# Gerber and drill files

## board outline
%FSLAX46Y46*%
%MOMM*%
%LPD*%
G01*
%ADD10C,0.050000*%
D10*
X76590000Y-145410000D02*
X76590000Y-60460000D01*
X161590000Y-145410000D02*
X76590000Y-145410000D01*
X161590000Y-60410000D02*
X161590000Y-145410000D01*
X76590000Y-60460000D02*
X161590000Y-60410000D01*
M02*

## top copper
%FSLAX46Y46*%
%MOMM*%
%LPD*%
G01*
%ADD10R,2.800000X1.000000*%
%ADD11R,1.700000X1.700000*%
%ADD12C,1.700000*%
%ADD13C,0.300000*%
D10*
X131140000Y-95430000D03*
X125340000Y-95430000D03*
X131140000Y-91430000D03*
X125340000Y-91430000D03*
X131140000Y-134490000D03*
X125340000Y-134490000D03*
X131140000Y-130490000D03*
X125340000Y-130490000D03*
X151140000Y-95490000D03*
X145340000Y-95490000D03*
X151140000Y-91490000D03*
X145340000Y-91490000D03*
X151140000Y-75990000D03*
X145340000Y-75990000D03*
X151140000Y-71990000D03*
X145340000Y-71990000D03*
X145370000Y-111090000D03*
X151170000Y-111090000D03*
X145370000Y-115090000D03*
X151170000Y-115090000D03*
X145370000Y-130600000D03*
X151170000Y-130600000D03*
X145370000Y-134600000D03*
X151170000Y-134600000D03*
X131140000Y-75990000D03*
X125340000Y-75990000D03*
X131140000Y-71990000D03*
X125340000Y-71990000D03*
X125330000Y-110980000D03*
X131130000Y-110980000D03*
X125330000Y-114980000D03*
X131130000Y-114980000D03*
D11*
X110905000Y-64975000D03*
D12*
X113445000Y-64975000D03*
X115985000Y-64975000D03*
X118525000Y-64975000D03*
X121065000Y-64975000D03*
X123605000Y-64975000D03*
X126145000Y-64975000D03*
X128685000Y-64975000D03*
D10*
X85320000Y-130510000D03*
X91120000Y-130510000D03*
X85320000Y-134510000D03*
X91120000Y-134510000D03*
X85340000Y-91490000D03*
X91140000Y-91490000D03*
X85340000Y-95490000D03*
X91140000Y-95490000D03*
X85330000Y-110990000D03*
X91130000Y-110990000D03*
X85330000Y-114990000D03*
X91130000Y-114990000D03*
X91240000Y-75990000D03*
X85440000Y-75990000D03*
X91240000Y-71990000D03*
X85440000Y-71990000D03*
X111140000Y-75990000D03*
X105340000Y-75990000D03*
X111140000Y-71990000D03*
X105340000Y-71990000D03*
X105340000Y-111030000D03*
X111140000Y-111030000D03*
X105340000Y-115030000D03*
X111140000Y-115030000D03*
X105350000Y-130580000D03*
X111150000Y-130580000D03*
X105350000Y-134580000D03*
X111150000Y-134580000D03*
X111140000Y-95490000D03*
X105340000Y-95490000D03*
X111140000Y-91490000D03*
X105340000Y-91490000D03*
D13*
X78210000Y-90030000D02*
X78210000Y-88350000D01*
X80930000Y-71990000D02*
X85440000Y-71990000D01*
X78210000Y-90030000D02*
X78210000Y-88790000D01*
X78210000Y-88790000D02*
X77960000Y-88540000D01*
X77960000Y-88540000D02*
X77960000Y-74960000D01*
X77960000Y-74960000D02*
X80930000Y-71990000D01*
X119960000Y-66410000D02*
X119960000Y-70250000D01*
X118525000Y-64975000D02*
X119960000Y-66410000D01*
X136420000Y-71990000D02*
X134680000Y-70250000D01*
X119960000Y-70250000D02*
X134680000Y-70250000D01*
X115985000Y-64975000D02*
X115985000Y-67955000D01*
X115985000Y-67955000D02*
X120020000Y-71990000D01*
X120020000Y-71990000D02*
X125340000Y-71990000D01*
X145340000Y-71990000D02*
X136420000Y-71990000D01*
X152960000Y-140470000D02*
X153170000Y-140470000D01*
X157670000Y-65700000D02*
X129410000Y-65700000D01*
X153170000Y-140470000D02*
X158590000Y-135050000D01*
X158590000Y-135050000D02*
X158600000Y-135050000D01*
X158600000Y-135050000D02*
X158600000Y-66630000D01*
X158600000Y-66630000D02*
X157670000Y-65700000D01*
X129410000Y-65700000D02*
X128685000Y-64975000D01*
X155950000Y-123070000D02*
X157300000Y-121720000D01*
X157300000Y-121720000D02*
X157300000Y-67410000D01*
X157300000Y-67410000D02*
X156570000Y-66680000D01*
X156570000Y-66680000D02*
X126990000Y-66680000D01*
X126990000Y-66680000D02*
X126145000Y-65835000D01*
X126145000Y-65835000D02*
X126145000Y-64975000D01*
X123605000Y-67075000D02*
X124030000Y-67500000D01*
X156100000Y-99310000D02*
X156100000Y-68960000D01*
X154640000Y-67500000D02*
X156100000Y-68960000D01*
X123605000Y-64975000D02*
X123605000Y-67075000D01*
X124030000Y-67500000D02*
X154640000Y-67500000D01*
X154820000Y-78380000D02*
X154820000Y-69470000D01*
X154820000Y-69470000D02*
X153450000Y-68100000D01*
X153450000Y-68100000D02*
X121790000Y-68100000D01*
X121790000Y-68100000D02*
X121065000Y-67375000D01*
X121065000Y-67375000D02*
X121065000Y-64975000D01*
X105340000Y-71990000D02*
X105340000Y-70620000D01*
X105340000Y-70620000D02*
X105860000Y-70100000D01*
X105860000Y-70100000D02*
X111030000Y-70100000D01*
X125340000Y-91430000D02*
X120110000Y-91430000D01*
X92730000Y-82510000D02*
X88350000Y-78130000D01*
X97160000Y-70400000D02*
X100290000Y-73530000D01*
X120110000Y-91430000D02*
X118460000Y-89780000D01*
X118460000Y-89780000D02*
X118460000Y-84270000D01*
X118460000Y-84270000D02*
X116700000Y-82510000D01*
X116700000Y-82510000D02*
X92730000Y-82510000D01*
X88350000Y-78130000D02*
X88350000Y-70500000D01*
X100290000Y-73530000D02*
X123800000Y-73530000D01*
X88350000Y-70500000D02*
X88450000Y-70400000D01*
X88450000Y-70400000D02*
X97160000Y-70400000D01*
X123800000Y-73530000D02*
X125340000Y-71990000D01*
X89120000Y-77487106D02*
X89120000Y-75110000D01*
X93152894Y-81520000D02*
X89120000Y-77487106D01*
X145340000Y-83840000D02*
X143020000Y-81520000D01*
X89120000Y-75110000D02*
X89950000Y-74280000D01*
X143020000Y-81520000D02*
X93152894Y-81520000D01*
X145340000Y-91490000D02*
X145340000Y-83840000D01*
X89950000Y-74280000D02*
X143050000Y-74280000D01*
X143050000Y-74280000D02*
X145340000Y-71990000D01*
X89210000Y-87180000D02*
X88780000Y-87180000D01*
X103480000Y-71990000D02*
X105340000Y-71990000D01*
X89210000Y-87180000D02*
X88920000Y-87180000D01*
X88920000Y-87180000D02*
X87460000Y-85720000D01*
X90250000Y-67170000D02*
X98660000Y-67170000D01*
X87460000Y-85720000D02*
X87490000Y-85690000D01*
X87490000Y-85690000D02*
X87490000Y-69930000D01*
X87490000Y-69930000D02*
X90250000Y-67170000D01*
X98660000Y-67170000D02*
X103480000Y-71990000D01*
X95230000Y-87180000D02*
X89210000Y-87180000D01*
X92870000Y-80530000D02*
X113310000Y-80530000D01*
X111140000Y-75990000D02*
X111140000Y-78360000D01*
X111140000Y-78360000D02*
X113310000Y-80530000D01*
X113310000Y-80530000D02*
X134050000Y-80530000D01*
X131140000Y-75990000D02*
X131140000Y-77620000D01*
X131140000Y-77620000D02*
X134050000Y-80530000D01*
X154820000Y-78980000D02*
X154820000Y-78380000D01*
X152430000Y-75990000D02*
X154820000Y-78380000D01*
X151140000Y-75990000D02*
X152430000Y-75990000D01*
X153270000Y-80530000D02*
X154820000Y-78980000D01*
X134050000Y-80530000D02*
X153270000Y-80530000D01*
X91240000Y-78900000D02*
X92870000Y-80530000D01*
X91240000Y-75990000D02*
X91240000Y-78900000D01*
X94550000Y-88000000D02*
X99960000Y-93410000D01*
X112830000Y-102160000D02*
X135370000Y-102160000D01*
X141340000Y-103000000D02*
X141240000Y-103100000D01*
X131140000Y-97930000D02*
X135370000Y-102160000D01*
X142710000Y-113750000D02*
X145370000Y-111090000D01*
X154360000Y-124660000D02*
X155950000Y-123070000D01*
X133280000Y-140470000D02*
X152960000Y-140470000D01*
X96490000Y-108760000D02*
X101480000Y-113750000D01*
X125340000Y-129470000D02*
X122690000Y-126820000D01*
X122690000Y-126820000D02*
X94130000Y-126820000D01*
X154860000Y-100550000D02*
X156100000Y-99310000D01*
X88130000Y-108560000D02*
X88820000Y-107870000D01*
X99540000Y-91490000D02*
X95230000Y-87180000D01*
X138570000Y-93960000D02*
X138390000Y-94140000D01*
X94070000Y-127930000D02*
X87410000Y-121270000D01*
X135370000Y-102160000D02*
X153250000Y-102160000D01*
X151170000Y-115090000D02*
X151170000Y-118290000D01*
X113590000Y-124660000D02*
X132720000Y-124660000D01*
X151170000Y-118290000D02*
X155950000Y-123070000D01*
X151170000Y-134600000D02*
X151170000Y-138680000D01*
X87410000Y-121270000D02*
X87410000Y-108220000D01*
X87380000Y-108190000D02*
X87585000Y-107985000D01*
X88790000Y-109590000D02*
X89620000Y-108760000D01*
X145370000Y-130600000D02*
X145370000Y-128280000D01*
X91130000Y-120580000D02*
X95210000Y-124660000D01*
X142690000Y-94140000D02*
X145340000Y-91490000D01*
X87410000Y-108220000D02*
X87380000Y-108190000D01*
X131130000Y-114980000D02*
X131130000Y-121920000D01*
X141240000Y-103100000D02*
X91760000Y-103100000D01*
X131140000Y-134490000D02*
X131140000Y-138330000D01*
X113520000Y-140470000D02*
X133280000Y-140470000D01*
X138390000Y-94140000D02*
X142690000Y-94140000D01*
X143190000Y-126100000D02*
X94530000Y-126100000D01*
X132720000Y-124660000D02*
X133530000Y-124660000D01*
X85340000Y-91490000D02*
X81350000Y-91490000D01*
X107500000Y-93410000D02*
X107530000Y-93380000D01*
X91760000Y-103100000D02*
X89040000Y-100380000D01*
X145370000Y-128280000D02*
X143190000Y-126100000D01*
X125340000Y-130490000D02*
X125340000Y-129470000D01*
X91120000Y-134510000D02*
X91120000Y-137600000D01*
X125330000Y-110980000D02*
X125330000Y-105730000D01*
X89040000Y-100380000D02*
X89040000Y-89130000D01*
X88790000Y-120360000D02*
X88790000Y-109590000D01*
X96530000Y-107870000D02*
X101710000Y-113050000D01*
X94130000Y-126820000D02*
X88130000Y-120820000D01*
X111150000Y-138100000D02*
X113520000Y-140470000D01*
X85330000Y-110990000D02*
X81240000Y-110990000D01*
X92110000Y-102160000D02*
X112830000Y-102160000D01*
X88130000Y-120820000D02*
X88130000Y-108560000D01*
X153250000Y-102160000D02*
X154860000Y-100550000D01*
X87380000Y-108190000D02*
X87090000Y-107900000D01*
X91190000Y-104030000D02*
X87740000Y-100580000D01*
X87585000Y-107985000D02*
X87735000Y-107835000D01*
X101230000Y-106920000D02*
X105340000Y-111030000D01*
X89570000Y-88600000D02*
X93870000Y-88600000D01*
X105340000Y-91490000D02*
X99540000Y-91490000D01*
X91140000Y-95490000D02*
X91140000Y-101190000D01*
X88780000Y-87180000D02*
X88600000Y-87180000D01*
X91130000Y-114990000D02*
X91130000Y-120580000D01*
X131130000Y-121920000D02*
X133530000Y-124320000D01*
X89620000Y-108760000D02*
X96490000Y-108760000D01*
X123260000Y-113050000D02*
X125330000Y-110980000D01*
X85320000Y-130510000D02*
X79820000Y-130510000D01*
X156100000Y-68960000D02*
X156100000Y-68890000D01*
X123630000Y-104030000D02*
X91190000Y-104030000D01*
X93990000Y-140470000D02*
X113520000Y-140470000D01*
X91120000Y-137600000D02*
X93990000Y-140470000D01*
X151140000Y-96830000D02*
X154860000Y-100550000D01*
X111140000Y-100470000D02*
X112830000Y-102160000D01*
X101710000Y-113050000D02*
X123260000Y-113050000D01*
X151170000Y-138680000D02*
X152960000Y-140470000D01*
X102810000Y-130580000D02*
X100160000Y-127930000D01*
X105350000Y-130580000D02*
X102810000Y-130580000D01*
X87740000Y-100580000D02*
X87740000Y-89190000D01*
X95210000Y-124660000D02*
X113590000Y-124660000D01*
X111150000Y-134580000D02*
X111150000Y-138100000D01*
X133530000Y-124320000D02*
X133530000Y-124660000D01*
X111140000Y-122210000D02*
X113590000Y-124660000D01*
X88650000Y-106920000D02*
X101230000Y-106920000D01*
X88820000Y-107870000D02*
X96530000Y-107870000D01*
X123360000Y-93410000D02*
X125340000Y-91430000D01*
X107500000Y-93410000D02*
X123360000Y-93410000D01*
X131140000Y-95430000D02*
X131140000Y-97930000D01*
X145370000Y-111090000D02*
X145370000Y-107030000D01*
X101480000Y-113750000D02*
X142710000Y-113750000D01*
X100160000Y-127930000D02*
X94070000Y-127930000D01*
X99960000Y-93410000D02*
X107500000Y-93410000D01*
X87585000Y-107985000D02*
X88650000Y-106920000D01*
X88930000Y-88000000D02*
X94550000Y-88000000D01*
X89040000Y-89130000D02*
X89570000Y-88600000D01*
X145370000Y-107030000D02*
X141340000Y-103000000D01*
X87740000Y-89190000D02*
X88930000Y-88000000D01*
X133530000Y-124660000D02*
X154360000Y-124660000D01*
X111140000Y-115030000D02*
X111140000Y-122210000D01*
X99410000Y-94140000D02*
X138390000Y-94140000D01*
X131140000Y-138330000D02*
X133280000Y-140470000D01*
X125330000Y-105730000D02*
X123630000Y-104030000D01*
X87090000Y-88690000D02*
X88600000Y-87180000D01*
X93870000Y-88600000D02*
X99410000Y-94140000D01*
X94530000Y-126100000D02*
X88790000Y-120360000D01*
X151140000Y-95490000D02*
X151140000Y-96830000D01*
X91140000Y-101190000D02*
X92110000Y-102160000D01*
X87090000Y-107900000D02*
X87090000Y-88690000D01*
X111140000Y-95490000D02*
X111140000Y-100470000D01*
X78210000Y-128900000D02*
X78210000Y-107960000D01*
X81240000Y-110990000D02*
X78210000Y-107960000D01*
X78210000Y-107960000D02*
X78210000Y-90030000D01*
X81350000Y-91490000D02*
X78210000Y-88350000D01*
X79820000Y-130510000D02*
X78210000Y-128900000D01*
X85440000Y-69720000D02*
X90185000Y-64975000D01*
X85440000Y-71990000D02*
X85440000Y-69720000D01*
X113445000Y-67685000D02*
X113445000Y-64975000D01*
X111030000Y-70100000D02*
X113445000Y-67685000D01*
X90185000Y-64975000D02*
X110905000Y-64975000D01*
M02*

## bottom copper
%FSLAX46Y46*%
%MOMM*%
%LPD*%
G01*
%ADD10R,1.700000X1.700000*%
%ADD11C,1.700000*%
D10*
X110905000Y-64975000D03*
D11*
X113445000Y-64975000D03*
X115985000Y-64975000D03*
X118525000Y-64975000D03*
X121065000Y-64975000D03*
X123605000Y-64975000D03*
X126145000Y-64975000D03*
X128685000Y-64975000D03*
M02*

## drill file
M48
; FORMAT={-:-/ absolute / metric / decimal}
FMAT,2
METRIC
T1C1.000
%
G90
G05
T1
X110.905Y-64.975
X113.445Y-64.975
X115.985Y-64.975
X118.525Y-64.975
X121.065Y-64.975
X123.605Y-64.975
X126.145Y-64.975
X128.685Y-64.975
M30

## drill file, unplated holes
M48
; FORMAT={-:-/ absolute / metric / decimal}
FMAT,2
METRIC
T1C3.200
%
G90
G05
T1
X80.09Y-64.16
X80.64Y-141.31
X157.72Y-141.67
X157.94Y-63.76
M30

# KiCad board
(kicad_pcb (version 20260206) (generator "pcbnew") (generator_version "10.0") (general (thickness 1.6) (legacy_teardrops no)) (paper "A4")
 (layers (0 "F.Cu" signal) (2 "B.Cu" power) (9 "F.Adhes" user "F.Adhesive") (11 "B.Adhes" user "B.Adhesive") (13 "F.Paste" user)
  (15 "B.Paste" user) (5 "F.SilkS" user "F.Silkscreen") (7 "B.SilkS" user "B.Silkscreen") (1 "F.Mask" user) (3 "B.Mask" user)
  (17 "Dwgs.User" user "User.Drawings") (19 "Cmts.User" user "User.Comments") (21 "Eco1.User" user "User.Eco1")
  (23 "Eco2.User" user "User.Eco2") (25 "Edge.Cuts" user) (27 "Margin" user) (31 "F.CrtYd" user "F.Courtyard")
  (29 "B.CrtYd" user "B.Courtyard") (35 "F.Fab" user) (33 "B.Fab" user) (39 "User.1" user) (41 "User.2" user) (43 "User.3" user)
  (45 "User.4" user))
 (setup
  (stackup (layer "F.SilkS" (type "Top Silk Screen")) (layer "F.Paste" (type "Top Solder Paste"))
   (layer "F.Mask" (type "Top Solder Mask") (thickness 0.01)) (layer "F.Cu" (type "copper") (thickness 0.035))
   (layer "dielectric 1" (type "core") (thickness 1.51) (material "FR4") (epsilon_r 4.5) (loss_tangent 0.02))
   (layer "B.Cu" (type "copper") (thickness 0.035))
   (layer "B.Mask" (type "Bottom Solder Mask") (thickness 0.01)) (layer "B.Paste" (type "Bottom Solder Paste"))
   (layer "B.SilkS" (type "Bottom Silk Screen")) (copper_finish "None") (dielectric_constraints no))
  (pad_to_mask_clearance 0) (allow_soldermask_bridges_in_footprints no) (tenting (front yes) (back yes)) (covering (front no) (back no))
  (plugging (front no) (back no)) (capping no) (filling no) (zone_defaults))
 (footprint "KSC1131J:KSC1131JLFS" (layer "F.Cu") (at 128.24 93.43)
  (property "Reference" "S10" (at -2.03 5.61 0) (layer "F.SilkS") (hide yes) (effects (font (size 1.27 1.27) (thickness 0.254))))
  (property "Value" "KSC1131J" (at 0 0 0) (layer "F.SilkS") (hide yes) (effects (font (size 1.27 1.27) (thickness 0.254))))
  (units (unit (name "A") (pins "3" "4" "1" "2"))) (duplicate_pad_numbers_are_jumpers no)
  (pad "1" smd rect (at -2.9 -2 90) (size 1 2.8) (layers "F.Cu" "F.Mask" "F.Paste") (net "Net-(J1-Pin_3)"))
  (pad "2" smd rect (at 2.9 -2 90) (size 1 2.8) (layers "F.Cu" "F.Mask" "F.Paste") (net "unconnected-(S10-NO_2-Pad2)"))
  (pad "3" smd rect (at -2.9 2 90) (size 1 2.8) (layers "F.Cu" "F.Mask" "F.Paste") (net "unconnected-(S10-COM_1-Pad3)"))
  (pad "4" smd rect (at 2.9 2 90) (size 1 2.8) (layers "F.Cu" "F.Mask" "F.Paste") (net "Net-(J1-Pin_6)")))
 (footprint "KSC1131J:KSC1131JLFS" (layer "F.Cu") (at 148.24 73.99)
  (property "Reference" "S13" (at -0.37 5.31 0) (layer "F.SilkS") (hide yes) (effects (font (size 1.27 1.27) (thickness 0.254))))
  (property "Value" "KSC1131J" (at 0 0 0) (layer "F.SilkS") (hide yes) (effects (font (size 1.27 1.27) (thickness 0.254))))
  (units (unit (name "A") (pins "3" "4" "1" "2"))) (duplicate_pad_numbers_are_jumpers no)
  (pad "1" smd rect (at -2.9 -2 90) (size 1 2.8) (layers "F.Cu" "F.Mask" "F.Paste") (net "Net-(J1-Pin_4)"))
  (pad "2" smd rect (at 2.9 -2 90) (size 1 2.8) (layers "F.Cu" "F.Mask" "F.Paste") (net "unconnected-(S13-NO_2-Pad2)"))
  (pad "3" smd rect (at -2.9 2 90) (size 1 2.8) (layers "F.Cu" "F.Mask" "F.Paste") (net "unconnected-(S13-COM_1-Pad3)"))
  (pad "4" smd rect (at 2.9 2 90) (size 1 2.8) (layers "F.Cu" "F.Mask" "F.Paste") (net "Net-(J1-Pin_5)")))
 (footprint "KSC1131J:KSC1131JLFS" (layer "F.Cu") (at 108.24 73.99)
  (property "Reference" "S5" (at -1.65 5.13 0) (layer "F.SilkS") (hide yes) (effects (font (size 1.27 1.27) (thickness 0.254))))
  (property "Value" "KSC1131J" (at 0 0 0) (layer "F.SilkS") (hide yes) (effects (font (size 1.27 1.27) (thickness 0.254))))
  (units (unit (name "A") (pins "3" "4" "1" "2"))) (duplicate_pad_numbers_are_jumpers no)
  (pad "1" smd rect (at -2.9 -2 90) (size 1 2.8) (layers "F.Cu" "F.Mask" "F.Paste") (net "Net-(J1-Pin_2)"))
  (pad "2" smd rect (at 2.9 -2 90) (size 1 2.8) (layers "F.Cu" "F.Mask" "F.Paste") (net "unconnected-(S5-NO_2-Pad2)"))
  (pad "3" smd rect (at -2.9 2 90) (size 1 2.8) (layers "F.Cu" "F.Mask" "F.Paste") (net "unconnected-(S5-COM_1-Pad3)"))
  (pad "4" smd rect (at 2.9 2 90) (size 1 2.8) (layers "F.Cu" "F.Mask" "F.Paste") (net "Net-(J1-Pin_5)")))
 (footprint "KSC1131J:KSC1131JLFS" (layer "F.Cu") (at 88.34 73.99)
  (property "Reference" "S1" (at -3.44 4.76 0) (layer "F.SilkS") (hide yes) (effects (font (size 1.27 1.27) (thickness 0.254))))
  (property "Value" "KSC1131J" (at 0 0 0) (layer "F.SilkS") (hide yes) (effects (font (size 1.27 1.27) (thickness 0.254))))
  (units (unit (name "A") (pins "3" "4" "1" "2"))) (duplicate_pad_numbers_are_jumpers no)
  (pad "1" smd rect (at -2.9 -2 90) (size 1 2.8) (layers "F.Cu" "F.Mask" "F.Paste") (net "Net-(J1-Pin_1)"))
  (pad "2" smd rect (at 2.9 -2 90) (size 1 2.8) (layers "F.Cu" "F.Mask" "F.Paste") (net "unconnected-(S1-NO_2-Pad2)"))
  (pad "3" smd rect (at -2.9 2 90) (size 1 2.8) (layers "F.Cu" "F.Mask" "F.Paste") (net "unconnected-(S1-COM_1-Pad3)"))
  (pad "4" smd rect (at 2.9 2 90) (size 1 2.8) (layers "F.Cu" "F.Mask" "F.Paste") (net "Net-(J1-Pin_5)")))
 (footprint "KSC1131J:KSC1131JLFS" (layer "F.Cu") (at 148.27 132.6)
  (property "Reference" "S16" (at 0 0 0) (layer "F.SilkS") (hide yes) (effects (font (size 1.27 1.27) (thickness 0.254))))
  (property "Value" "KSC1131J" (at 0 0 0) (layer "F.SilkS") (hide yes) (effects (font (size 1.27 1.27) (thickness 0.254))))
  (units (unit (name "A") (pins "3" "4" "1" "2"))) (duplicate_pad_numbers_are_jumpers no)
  (pad "1" smd rect (at -2.9 -2 90) (size 1 2.8) (layers "F.Cu" "F.Mask" "F.Paste") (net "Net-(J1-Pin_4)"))
  (pad "2" smd rect (at 2.9 -2 90) (size 1 2.8) (layers "F.Cu" "F.Mask" "F.Paste") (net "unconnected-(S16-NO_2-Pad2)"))
  (pad "3" smd rect (at -2.9 2 90) (size 1 2.8) (layers "F.Cu" "F.Mask" "F.Paste") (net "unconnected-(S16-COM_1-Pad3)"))
  (pad "4" smd rect (at 2.9 2 90) (size 1 2.8) (layers "F.Cu" "F.Mask" "F.Paste") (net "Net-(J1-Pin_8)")))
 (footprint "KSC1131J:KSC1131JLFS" (layer "F.Cu") (at 128.24 73.99)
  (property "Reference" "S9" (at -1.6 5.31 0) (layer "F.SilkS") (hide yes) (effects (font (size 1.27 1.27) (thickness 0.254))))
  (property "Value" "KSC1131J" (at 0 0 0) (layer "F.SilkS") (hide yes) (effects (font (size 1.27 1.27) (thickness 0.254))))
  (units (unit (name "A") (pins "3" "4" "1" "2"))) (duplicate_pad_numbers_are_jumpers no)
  (pad "1" smd rect (at -2.9 -2 90) (size 1 2.8) (layers "F.Cu" "F.Mask" "F.Paste") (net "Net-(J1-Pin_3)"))
  (pad "2" smd rect (at 2.9 -2 90) (size 1 2.8) (layers "F.Cu" "F.Mask" "F.Paste") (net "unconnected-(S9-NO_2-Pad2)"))
  (pad "3" smd rect (at -2.9 2 90) (size 1 2.8) (layers "F.Cu" "F.Mask" "F.Paste") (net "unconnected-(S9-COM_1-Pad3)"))
  (pad "4" smd rect (at 2.9 2 90) (size 1 2.8) (layers "F.Cu" "F.Mask" "F.Paste") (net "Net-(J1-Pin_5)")))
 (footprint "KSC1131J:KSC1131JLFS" (layer "F.Cu") (at 108.24 93.49)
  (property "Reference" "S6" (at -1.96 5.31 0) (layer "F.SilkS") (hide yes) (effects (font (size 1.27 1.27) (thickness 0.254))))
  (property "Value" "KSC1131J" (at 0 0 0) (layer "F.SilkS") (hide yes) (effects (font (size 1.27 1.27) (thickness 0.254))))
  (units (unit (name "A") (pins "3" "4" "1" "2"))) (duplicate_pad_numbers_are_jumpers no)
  (pad "1" smd rect (at -2.9 -2 90) (size 1 2.8) (layers "F.Cu" "F.Mask" "F.Paste") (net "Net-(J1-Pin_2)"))
  (pad "2" smd rect (at 2.9 -2 90) (size 1 2.8) (layers "F.Cu" "F.Mask" "F.Paste") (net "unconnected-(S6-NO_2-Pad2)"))
  (pad "3" smd rect (at -2.9 2 90) (size 1 2.8) (layers "F.Cu" "F.Mask" "F.Paste") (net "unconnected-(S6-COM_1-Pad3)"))
  (pad "4" smd rect (at 2.9 2 90) (size 1 2.8) (layers "F.Cu" "F.Mask" "F.Paste") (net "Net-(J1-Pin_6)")))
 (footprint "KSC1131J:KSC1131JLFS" (layer "F.Cu") (at 148.27 113.09)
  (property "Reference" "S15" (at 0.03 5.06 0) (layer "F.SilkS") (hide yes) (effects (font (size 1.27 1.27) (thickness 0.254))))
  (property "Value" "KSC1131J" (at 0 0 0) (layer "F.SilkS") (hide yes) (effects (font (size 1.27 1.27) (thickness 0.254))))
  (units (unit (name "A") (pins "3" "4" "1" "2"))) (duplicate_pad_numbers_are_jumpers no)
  (pad "1" smd rect (at -2.9 -2 90) (size 1 2.8) (layers "F.Cu" "F.Mask" "F.Paste") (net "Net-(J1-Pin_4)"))
  (pad "2" smd rect (at 2.9 -2 90) (size 1 2.8) (layers "F.Cu" "F.Mask" "F.Paste") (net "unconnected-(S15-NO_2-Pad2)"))
  (pad "3" smd rect (at -2.9 2 90) (size 1 2.8) (layers "F.Cu" "F.Mask" "F.Paste") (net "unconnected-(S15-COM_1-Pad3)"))
  (pad "4" smd rect (at 2.9 2 90) (size 1 2.8) (layers "F.Cu" "F.Mask" "F.Paste") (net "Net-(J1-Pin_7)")))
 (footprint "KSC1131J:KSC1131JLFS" (layer "F.Cu") (at 108.24 113.03)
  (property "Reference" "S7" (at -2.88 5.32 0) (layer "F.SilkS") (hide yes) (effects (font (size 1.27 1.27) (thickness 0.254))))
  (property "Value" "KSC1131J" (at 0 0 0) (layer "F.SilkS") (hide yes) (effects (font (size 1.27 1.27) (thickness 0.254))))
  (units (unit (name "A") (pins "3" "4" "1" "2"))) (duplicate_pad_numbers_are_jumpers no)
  (pad "1" smd rect (at -2.9 -2 90) (size 1 2.8) (layers "F.Cu" "F.Mask" "F.Paste") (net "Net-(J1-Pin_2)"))
  (pad "2" smd rect (at 2.9 -2 90) (size 1 2.8) (layers "F.Cu" "F.Mask" "F.Paste") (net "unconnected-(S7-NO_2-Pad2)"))
  (pad "3" smd rect (at -2.9 2 90) (size 1 2.8) (layers "F.Cu" "F.Mask" "F.Paste") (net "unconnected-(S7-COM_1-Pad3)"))
  (pad "4" smd rect (at 2.9 2 90) (size 1 2.8) (layers "F.Cu" "F.Mask" "F.Paste") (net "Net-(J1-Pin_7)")))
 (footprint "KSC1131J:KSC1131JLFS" (layer "F.Cu") (at 148.24 93.49)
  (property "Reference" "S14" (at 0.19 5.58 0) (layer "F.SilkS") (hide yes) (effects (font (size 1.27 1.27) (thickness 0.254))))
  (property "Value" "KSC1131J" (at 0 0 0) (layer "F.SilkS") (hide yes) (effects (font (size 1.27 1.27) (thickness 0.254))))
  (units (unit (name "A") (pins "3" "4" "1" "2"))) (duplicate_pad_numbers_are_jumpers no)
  (pad "1" smd rect (at -2.9 -2 90) (size 1 2.8) (layers "F.Cu" "F.Mask" "F.Paste") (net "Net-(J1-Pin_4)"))
  (pad "2" smd rect (at 2.9 -2 90) (size 1 2.8) (layers "F.Cu" "F.Mask" "F.Paste") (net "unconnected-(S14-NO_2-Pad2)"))
  (pad "3" smd rect (at -2.9 2 90) (size 1 2.8) (layers "F.Cu" "F.Mask" "F.Paste") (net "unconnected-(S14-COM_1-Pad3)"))
  (pad "4" smd rect (at 2.9 2 90) (size 1 2.8) (layers "F.Cu" "F.Mask" "F.Paste") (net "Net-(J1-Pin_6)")))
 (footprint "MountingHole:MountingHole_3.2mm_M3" (layer "F.Cu") (at 157.72 141.67)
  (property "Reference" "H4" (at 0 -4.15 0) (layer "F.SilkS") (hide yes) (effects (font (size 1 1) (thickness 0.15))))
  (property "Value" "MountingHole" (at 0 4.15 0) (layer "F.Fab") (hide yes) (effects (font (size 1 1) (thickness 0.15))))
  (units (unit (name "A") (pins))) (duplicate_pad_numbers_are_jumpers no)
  (pad "" np_thru_hole circle (at 0 0) (size 3.2 3.2) (drill 3.2) (layers "*.Cu" "*.Mask")))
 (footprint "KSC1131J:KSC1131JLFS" (layer "F.Cu") (at 128.24 132.49)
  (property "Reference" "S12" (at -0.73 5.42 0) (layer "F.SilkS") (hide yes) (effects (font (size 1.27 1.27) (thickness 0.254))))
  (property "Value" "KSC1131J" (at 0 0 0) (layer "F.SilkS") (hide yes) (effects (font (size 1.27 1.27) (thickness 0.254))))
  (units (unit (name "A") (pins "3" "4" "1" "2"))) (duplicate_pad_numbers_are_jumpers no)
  (pad "1" smd rect (at -2.9 -2 90) (size 1 2.8) (layers "F.Cu" "F.Mask" "F.Paste") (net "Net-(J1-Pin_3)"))
  (pad "2" smd rect (at 2.9 -2 90) (size 1 2.8) (layers "F.Cu" "F.Mask" "F.Paste") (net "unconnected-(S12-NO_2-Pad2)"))
  (pad "3" smd rect (at -2.9 2 90) (size 1 2.8) (layers "F.Cu" "F.Mask" "F.Paste") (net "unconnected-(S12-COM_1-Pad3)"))
  (pad "4" smd rect (at 2.9 2 90) (size 1 2.8) (layers "F.Cu" "F.Mask" "F.Paste") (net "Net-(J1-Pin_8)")))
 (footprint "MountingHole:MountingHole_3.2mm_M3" (layer "F.Cu") (at 157.94 63.76)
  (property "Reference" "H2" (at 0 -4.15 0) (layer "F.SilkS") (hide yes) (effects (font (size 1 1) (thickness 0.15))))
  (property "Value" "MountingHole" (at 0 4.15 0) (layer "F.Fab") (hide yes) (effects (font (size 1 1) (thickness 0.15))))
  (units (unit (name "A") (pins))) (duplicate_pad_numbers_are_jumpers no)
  (pad "" np_thru_hole circle (at 0 0) (size 3.2 3.2) (drill 3.2) (layers "*.Cu" "*.Mask")))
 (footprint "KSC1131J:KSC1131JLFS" (layer "F.Cu") (at 88.23 112.99)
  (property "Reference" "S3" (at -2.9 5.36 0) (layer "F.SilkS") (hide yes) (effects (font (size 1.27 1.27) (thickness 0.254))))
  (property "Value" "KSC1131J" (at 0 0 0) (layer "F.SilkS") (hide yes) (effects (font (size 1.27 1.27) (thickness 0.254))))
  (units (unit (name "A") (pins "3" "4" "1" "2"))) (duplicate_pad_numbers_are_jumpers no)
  (pad "1" smd rect (at -2.9 -2 90) (size 1 2.8) (layers "F.Cu" "F.Mask" "F.Paste") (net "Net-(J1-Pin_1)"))
  (pad "2" smd rect (at 2.9 -2 90) (size 1 2.8) (layers "F.Cu" "F.Mask" "F.Paste") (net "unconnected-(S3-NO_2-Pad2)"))
  (pad "3" smd rect (at -2.9 2 90) (size 1 2.8) (layers "F.Cu" "F.Mask" "F.Paste") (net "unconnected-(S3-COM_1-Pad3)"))
  (pad "4" smd rect (at 2.9 2 90) (size 1 2.8) (layers "F.Cu" "F.Mask" "F.Paste") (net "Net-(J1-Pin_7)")))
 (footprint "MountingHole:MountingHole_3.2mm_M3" (layer "F.Cu") (at 80.64 141.31)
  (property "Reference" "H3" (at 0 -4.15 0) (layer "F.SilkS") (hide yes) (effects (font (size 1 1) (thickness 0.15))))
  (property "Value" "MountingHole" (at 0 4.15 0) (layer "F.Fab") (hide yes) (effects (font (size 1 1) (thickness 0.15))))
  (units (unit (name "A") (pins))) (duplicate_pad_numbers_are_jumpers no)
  (pad "" np_thru_hole circle (at 0 0) (size 3.2 3.2) (drill 3.2) (layers "*.Cu" "*.Mask")))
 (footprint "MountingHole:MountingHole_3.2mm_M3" (layer "F.Cu") (at 80.09 64.16)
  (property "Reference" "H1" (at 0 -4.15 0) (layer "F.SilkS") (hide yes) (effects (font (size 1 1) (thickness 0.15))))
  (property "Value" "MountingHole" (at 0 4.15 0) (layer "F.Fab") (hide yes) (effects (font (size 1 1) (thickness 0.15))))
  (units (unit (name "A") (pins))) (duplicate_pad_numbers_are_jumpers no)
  (pad "" np_thru_hole circle (at 0 0) (size 3.2 3.2) (drill 3.2) (layers "*.Cu" "*.Mask")))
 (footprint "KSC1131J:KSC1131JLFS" (layer "F.Cu") (at 88.24 93.49)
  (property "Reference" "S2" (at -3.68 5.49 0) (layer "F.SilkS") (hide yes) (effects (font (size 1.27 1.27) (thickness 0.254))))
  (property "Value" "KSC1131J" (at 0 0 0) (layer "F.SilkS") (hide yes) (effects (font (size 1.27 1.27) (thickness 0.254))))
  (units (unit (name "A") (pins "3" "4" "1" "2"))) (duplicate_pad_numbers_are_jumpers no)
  (pad "1" smd rect (at -2.9 -2 90) (size 1 2.8) (layers "F.Cu" "F.Mask" "F.Paste") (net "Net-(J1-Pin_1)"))
  (pad "2" smd rect (at 2.9 -2 90) (size 1 2.8) (layers "F.Cu" "F.Mask" "F.Paste") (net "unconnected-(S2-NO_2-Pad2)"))
  (pad "3" smd rect (at -2.9 2 90) (size 1 2.8) (layers "F.Cu" "F.Mask" "F.Paste") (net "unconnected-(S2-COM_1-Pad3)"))
  (pad "4" smd rect (at 2.9 2 90) (size 1 2.8) (layers "F.Cu" "F.Mask" "F.Paste") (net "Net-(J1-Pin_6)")))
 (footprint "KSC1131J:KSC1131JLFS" (layer "F.Cu") (at 128.23 112.98)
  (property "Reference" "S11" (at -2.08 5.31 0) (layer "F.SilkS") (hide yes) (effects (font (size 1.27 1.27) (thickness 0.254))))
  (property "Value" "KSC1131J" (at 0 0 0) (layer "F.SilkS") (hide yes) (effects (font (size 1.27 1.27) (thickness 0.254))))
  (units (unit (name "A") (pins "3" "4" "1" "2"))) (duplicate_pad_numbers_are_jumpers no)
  (pad "1" smd rect (at -2.9 -2 90) (size 1 2.8) (layers "F.Cu" "F.Mask" "F.Paste") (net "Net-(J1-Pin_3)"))
  (pad "2" smd rect (at 2.9 -2 90) (size 1 2.8) (layers "F.Cu" "F.Mask" "F.Paste") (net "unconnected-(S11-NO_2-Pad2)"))
  (pad "3" smd rect (at -2.9 2 90) (size 1 2.8) (layers "F.Cu" "F.Mask" "F.Paste") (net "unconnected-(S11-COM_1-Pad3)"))
  (pad "4" smd rect (at 2.9 2 90) (size 1 2.8) (layers "F.Cu" "F.Mask" "F.Paste") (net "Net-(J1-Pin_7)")))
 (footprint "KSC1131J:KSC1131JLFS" (layer "F.Cu") (at 88.22 132.51)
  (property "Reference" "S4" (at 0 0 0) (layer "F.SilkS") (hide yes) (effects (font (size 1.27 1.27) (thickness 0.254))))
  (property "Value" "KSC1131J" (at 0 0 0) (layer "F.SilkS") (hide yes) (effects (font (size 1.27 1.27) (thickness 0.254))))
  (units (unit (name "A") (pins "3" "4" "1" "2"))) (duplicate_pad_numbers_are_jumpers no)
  (pad "1" smd rect (at -2.9 -2 90) (size 1 2.8) (layers "F.Cu" "F.Mask" "F.Paste") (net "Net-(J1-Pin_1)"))
  (pad "2" smd rect (at 2.9 -2 90) (size 1 2.8) (layers "F.Cu" "F.Mask" "F.Paste") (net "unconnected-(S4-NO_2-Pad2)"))
  (pad "3" smd rect (at -2.9 2 90) (size 1 2.8) (layers "F.Cu" "F.Mask" "F.Paste") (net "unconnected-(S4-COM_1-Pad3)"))
  (pad "4" smd rect (at 2.9 2 90) (size 1 2.8) (layers "F.Cu" "F.Mask" "F.Paste") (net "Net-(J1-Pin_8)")))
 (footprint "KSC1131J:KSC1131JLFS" (layer "F.Cu") (at 108.25 132.58)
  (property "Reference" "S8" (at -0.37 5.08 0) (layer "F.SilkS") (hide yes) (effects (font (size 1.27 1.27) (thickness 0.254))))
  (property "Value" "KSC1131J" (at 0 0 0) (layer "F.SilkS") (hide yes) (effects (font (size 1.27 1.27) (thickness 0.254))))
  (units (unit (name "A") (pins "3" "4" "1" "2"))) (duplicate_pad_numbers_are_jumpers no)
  (pad "1" smd rect (at -2.9 -2 90) (size 1 2.8) (layers "F.Cu" "F.Mask" "F.Paste") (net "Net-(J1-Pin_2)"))
  (pad "2" smd rect (at 2.9 -2 90) (size 1 2.8) (layers "F.Cu" "F.Mask" "F.Paste") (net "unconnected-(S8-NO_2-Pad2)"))
  (pad "3" smd rect (at -2.9 2 90) (size 1 2.8) (layers "F.Cu" "F.Mask" "F.Paste") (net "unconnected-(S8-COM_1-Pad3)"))
  (pad "4" smd rect (at 2.9 2 90) (size 1 2.8) (layers "F.Cu" "F.Mask" "F.Paste") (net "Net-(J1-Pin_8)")))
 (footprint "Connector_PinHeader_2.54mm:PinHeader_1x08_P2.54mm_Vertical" (layer "F.Cu") (at 110.905 64.975 90)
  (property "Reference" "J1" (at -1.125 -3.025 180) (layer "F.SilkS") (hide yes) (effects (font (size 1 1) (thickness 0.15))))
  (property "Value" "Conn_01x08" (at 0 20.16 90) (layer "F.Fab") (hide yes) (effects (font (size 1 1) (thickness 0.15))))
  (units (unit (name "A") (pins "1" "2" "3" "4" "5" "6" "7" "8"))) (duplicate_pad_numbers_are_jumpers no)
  (pad "1" thru_hole rect (at 0 0 90) (size 1.7 1.7) (drill 1) (layers "*.Cu" "*.Mask") (remove_unused_layers no) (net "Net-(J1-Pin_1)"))
  (pad "2" thru_hole circle (at 0 2.54 90) (size 1.7 1.7) (drill 1) (layers "*.Cu" "*.Mask") (remove_unused_layers no)
   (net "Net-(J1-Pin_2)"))
  (pad "3" thru_hole circle (at 0 5.08 90) (size 1.7 1.7) (drill 1) (layers "*.Cu" "*.Mask") (remove_unused_layers no)
   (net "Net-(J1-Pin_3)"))
  (pad "4" thru_hole circle (at 0 7.62 90) (size 1.7 1.7) (drill 1) (layers "*.Cu" "*.Mask") (remove_unused_layers no)
   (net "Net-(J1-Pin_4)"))
  (pad "5" thru_hole circle (at 0 10.16 90) (size 1.7 1.7) (drill 1) (layers "*.Cu" "*.Mask") (remove_unused_layers no)
   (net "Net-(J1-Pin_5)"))
  (pad "6" thru_hole circle (at 0 12.7 90) (size 1.7 1.7) (drill 1) (layers "*.Cu" "*.Mask") (remove_unused_layers no)
   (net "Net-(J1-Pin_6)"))
  (pad "7" thru_hole circle (at 0 15.24 90) (size 1.7 1.7) (drill 1) (layers "*.Cu" "*.Mask") (remove_unused_layers no)
   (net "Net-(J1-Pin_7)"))
  (pad "8" thru_hole circle (at 0 17.78 90) (size 1.7 1.7) (drill 1) (layers "*.Cu" "*.Mask") (remove_unused_layers no)
   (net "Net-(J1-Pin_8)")))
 (gr_line (start 76.59 60.46) (end 161.59 60.41) (stroke (width 0.05) (type default)) (layer "Edge.Cuts"))
 (gr_line (start 76.59 145.41) (end 76.59 60.46) (stroke (width 0.05) (type default)) (layer "Edge.Cuts"))
 (gr_line (start 161.59 60.41) (end 161.59 145.41) (stroke (width 0.05) (type default)) (layer "Edge.Cuts"))
 (gr_line (start 161.59 145.41) (end 76.59 145.41) (stroke (width 0.05) (type default)) (layer "Edge.Cuts"))
 (segment (start 85.34 91.49) (end 81.35 91.49) (width 0.3) (layer "F.Cu") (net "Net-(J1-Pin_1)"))
 (segment (start 85.44 69.72) (end 90.185 64.975) (width 0.3) (layer "F.Cu") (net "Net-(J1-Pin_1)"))
 (segment (start 79.82 130.51) (end 78.21 128.9) (width 0.3) (layer "F.Cu") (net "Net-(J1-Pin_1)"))
 (segment (start 78.21 128.9) (end 78.21 107.96) (width 0.3) (layer "F.Cu") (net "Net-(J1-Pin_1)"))
 (segment (start 85.33 110.99) (end 81.24 110.99) (width 0.3) (layer "F.Cu") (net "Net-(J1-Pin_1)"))
 (segment (start 78.21 88.79) (end 77.96 88.54) (width 0.3) (layer "F.Cu") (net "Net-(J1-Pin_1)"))
 (segment (start 85.32 130.51) (end 79.82 130.51) (width 0.3) (layer "F.Cu") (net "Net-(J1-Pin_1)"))
 (segment (start 77.96 88.54) (end 77.96 74.96) (width 0.3) (layer "F.Cu") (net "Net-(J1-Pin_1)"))
 (segment (start 81.35 91.49) (end 78.21 88.35) (width 0.3) (layer "F.Cu") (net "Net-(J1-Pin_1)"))
 (segment (start 78.21 90.03) (end 78.21 88.79) (width 0.3) (layer "F.Cu") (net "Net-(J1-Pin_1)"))
 (segment (start 78.21 107.96) (end 78.21 90.03) (width 0.3) (layer "F.Cu") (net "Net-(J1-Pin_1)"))
 (segment (start 80.93 71.99) (end 85.44 71.99) (width 0.3) (layer "F.Cu") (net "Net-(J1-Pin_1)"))
 (segment (start 90.185 64.975) (end 110.905 64.975) (width 0.3) (layer "F.Cu") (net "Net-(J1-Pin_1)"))
 (segment (start 78.21 90.03) (end 78.21 88.35) (width 0.3) (layer "F.Cu") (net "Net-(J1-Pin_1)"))
 (segment (start 77.96 74.96) (end 80.93 71.99) (width 0.3) (layer "F.Cu") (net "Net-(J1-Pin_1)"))
 (segment (start 81.24 110.99) (end 78.21 107.96) (width 0.3) (layer "F.Cu") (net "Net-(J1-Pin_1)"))
 (segment (start 85.44 71.99) (end 85.44 69.72) (width 0.3) (layer "F.Cu") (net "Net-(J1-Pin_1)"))
 (segment (start 87.09 107.9) (end 87.09 88.69) (width 0.3) (layer "F.Cu") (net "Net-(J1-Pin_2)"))
 (segment (start 87.41 121.27) (end 87.41 108.22) (width 0.3) (layer "F.Cu") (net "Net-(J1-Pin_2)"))
 (segment (start 87.585 107.985) (end 87.735 107.835) (width 0.3) (layer "F.Cu") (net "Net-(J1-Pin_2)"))
 (segment (start 113.445 67.685) (end 113.445 64.975) (width 0.3) (layer "F.Cu") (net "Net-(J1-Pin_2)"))
 (segment (start 90.25 67.17) (end 98.66 67.17) (width 0.3) (layer "F.Cu") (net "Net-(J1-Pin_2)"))
 (segment (start 89.21 87.18) (end 88.78 87.18) (width 0.3) (layer "F.Cu") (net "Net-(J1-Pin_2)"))
 (segment (start 88.78 87.18) (end 88.6 87.18) (width 0.3) (layer "F.Cu") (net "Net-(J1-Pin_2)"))
 (segment (start 103.48 71.99) (end 105.34 71.99) (width 0.3) (layer "F.Cu") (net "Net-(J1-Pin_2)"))
 (segment (start 87.585 107.985) (end 88.65 106.92) (width 0.3) (layer "F.Cu") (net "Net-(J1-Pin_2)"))
 (segment (start 94.07 127.93) (end 87.41 121.27) (width 0.3) (layer "F.Cu") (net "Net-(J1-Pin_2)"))
 (segment (start 102.81 130.58) (end 100.16 127.93) (width 0.3) (layer "F.Cu") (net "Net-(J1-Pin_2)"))
 (segment (start 111.03 70.1) (end 113.445 67.685) (width 0.3) (layer "F.Cu") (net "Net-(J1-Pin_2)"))
 (segment (start 87.38 108.19) (end 87.09 107.9) (width 0.3) (layer "F.Cu") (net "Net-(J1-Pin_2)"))
 (segment (start 105.35 130.58) (end 102.81 130.58) (width 0.3) (layer "F.Cu") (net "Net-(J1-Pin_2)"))
 (segment (start 89.21 87.18) (end 88.92 87.18) (width 0.3) (layer "F.Cu") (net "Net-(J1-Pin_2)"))
 (segment (start 101.23 106.92) (end 105.34 111.03) (width 0.3) (layer "F.Cu") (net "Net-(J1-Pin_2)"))
 (segment (start 88.65 106.92) (end 101.23 106.92) (width 0.3) (layer "F.Cu") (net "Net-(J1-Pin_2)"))
 (segment (start 87.49 85.69) (end 87.49 69.93) (width 0.3) (layer "F.Cu") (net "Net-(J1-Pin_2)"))
 (segment (start 105.86 70.1) (end 111.03 70.1) (width 0.3) (layer "F.Cu") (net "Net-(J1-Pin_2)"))
 (segment (start 100.16 127.93) (end 94.07 127.93) (width 0.3) (layer "F.Cu") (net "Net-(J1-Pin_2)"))
 (segment (start 87.41 108.22) (end 87.38 108.19) (width 0.3) (layer "F.Cu") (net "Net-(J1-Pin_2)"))
 (segment (start 87.49 69.93) (end 90.25 67.17) (width 0.3) (layer "F.Cu") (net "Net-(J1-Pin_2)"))
 (segment (start 87.09 88.69) (end 88.6 87.18) (width 0.3) (layer "F.Cu") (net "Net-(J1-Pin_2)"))
 (segment (start 99.54 91.49) (end 95.23 87.18) (width 0.3) (layer "F.Cu") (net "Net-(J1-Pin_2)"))
 (segment (start 105.34 91.49) (end 99.54 91.49) (width 0.3) (layer "F.Cu") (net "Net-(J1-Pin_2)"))
 (segment (start 105.34 70.62) (end 105.86 70.1) (width 0.3) (layer "F.Cu") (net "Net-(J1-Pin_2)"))
 (segment (start 98.66 67.17) (end 103.48 71.99) (width 0.3) (layer "F.Cu") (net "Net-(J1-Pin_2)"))
 (segment (start 87.46 85.72) (end 87.49 85.69) (width 0.3) (layer "F.Cu") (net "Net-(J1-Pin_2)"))
 (segment (start 105.34 71.99) (end 105.34 70.62) (width 0.3) (layer "F.Cu") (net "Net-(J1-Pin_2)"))
 (segment (start 87.38 108.19) (end 87.585 107.985) (width 0.3) (layer "F.Cu") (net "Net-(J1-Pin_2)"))
 (segment (start 88.92 87.18) (end 87.46 85.72) (width 0.3) (layer "F.Cu") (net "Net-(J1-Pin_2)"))
 (segment (start 95.23 87.18) (end 89.21 87.18) (width 0.3) (layer "F.Cu") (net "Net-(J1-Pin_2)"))
 (segment (start 92.73 82.51) (end 88.35 78.13) (width 0.3) (layer "F.Cu") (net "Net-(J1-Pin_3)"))
 (segment (start 88.82 107.87) (end 96.53 107.87) (width 0.3) (layer "F.Cu") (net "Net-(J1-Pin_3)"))
 (segment (start 88.93 88) (end 94.55 88) (width 0.3) (layer "F.Cu") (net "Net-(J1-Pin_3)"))
 (segment (start 125.34 130.49) (end 125.34 129.47) (width 0.3) (layer "F.Cu") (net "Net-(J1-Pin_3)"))
 (segment (start 118.46 84.27) (end 116.7 82.51) (width 0.3) (layer "F.Cu") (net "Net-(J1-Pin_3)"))
 (segment (start 120.02 71.99) (end 125.34 71.99) (width 0.3) (layer "F.Cu") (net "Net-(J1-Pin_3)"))
 (segment (start 94.55 88) (end 99.96 93.41) (width 0.3) (layer "F.Cu") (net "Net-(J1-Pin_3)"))
 (segment (start 96.53 107.87) (end 101.71 113.05) (width 0.3) (layer "F.Cu") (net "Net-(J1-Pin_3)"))
 (segment (start 88.35 70.5) (end 88.45 70.4) (width 0.3) (layer "F.Cu") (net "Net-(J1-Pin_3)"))
 (segment (start 115.985 64.975) (end 115.985 67.955) (width 0.3) (layer "F.Cu") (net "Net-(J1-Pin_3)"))
 (segment (start 115.985 67.955) (end 120.02 71.99) (width 0.3) (layer "F.Cu") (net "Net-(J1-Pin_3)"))
 (segment (start 122.69 126.82) (end 94.13 126.82) (width 0.3) (layer "F.Cu") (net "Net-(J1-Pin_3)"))
 (segment (start 125.34 91.43) (end 120.11 91.43) (width 0.3) (layer "F.Cu") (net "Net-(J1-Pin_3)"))
 (segment (start 107.5 93.41) (end 107.53 93.38) (width 0.3) (layer "F.Cu") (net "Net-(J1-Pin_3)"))
 (segment (start 88.45 70.4) (end 97.16 70.4) (width 0.3) (layer "F.Cu") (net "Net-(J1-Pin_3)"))
 (segment (start 118.46 89.78) (end 118.46 84.27) (width 0.3) (layer "F.Cu") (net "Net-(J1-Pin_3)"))
 (segment (start 99.96 93.41) (end 107.5 93.41) (width 0.3) (layer "F.Cu") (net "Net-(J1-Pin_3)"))
 (segment (start 88.35 78.13) (end 88.35 70.5) (width 0.3) (layer "F.Cu") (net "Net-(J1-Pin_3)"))
 (segment (start 123.26 113.05) (end 125.33 110.98) (width 0.3) (layer "F.Cu") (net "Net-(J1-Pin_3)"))
 (segment (start 94.13 126.82) (end 88.13 120.82) (width 0.3) (layer "F.Cu") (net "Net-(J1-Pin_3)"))
 (segment (start 123.36 93.41) (end 125.34 91.43) (width 0.3) (layer "F.Cu") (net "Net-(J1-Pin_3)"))
 (segment (start 91.19 104.03) (end 87.74 100.58) (width 0.3) (layer "F.Cu") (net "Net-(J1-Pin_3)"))
 (segment (start 125.34 129.47) (end 122.69 126.82) (width 0.3) (layer "F.Cu") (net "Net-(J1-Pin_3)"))
 (segment (start 88.13 120.82) (end 88.13 108.56) (width 0.3) (layer "F.Cu") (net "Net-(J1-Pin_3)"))
 (segment (start 107.5 93.41) (end 123.36 93.41) (width 0.3) (layer "F.Cu") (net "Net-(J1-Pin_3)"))
 (segment (start 101.71 113.05) (end 123.26 113.05) (width 0.3) (layer "F.Cu") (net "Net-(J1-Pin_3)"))
 (segment (start 87.74 100.58) (end 87.74 89.19) (width 0.3) (layer "F.Cu") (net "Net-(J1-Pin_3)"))
 (segment (start 123.8 73.53) (end 125.34 71.99) (width 0.3) (layer "F.Cu") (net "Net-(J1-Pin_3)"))
 (segment (start 116.7 82.51) (end 92.73 82.51) (width 0.3) (layer "F.Cu") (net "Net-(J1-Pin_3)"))
 (segment (start 125.33 105.73) (end 123.63 104.03) (width 0.3) (layer "F.Cu") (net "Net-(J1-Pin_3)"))
 (segment (start 87.74 89.19) (end 88.93 88) (width 0.3) (layer "F.Cu") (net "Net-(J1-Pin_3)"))
 (segment (start 97.16 70.4) (end 100.29 73.53) (width 0.3) (layer "F.Cu") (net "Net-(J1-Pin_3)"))
 (segment (start 88.13 108.56) (end 88.82 107.87) (width 0.3) (layer "F.Cu") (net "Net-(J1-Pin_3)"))
 (segment (start 125.33 110.98) (end 125.33 105.73) (width 0.3) (layer "F.Cu") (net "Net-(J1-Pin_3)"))
 (segment (start 120.11 91.43) (end 118.46 89.78) (width 0.3) (layer "F.Cu") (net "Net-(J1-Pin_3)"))
 (segment (start 123.63 104.03) (end 91.19 104.03) (width 0.3) (layer "F.Cu") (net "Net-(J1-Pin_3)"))
 (segment (start 100.29 73.53) (end 123.8 73.53) (width 0.3) (layer "F.Cu") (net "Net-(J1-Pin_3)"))
 (segment (start 91.24 75.99) (end 91.24 78.9) (width 0.3) (layer "F.Cu") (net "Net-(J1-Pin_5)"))
 (segment (start 121.79 68.1) (end 121.065 67.375) (width 0.3) (layer "F.Cu") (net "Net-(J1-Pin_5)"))
 (segment (start 131.14 77.62) (end 134.05 80.53) (width 0.3) (layer "F.Cu") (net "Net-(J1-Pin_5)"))
 (segment (start 121.065 67.375) (end 121.065 64.975) (width 0.3) (layer "F.Cu") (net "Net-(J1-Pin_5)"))
 (segment (start 154.82 78.98) (end 154.82 78.38) (width 0.3) (layer "F.Cu") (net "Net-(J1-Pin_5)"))
 (segment (start 154.82 69.47) (end 153.45 68.1) (width 0.3) (layer "F.Cu") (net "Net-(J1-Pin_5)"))
 (segment (start 111.14 78.36) (end 113.31 80.53) (width 0.3) (layer "F.Cu") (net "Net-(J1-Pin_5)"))
 (segment (start 113.31 80.53) (end 134.05 80.53) (width 0.3) (layer "F.Cu") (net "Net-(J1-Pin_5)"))
 (segment (start 91.24 78.9) (end 92.87 80.53) (width 0.3) (layer "F.Cu") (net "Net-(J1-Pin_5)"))
 (segment (start 92.87 80.53) (end 113.31 80.53) (width 0.3) (layer "F.Cu") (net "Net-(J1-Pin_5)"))
 (segment (start 134.05 80.53) (end 153.27 80.53) (width 0.3) (layer "F.Cu") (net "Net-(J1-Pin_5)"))
 (segment (start 153.27 80.53) (end 154.82 78.98) (width 0.3) (layer "F.Cu") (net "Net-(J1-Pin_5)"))
 (segment (start 154.82 78.38) (end 154.82 69.47) (width 0.3) (layer "F.Cu") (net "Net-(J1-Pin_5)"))
 (segment (start 131.14 75.99) (end 131.14 77.62) (width 0.3) (layer "F.Cu") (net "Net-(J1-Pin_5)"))
 (segment (start 153.45 68.1) (end 121.79 68.1) (width 0.3) (layer "F.Cu") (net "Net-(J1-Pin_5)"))
 (segment (start 111.14 75.99) (end 111.14 78.36) (width 0.3) (layer "F.Cu") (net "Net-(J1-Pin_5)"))
 (segment (start 151.14 75.99) (end 152.43 75.99) (width 0.3) (layer "F.Cu") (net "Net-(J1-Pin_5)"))
 (segment (start 152.43 75.99) (end 154.82 78.38) (width 0.3) (layer "F.Cu") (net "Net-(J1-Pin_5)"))
 (segment (start 112.83 102.16) (end 135.37 102.16) (width 0.3) (layer "F.Cu") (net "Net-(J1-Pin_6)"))
 (segment (start 124.03 67.5) (end 154.64 67.5) (width 0.3) (layer "F.Cu") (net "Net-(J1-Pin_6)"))
 (segment (start 153.25 102.16) (end 154.86 100.55) (width 0.3) (layer "F.Cu") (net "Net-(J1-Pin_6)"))
 (segment (start 91.14 95.49) (end 91.14 101.19) (width 0.3) (layer "F.Cu") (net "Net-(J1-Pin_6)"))
 (segment (start 111.14 100.47) (end 112.83 102.16) (width 0.3) (layer "F.Cu") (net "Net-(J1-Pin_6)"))
 (segment (start 123.605 67.075) (end 124.03 67.5) (width 0.3) (layer "F.Cu") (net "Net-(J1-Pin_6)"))
 (segment (start 151.14 96.83) (end 154.86 100.55) (width 0.3) (layer "F.Cu") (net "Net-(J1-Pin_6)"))
 (segment (start 135.37 102.16) (end 153.25 102.16) (width 0.3) (layer "F.Cu") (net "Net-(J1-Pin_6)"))
 (segment (start 123.605 64.975) (end 123.605 67.075) (width 0.3) (layer "F.Cu") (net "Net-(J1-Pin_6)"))
 (segment (start 92.11 102.16) (end 112.83 102.16) (width 0.3) (layer "F.Cu") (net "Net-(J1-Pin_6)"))
 (segment (start 154.86 100.55) (end 156.1 99.31) (width 0.3) (layer "F.Cu") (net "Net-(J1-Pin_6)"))
 (segment (start 151.14 95.49) (end 151.14 96.83) (width 0.3) (layer "F.Cu") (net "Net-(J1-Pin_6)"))
 (segment (start 154.64 67.5) (end 156.1 68.96) (width 0.3) (layer "F.Cu") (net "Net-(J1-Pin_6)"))
 (segment (start 111.14 95.49) (end 111.14 100.47) (width 0.3) (layer "F.Cu") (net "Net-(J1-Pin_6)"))
 (segment (start 131.14 97.93) (end 135.37 102.16) (width 0.3) (layer "F.Cu") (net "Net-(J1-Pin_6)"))
 (segment (start 91.14 101.19) (end 92.11 102.16) (width 0.3) (layer "F.Cu") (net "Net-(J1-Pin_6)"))
 (segment (start 131.14 95.43) (end 131.14 97.93) (width 0.3) (layer "F.Cu") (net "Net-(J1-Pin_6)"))
 (segment (start 156.1 99.31) (end 156.1 68.96) (width 0.3) (layer "F.Cu") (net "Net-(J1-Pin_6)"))
 (segment (start 156.1 68.96) (end 156.1 68.89) (width 0.3) (layer "F.Cu") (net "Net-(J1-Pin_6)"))
 (segment (start 95.21 124.66) (end 113.59 124.66) (width 0.3) (layer "F.Cu") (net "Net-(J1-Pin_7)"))
 (segment (start 132.72 124.66) (end 133.53 124.66) (width 0.3) (layer "F.Cu") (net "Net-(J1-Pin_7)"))
 (segment (start 91.13 120.58) (end 95.21 124.66) (width 0.3) (layer "F.Cu") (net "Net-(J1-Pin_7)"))
 (segment (start 113.59 124.66) (end 132.72 124.66) (width 0.3) (layer "F.Cu") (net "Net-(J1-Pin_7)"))
 (segment (start 126.145 65.835) (end 126.145 64.975) (width 0.3) (layer "F.Cu") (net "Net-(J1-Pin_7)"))
 (segment (start 131.13 114.98) (end 131.13 121.92) (width 0.3) (layer "F.Cu") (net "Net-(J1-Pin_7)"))
 (segment (start 111.14 122.21) (end 113.59 124.66) (width 0.3) (layer "F.Cu") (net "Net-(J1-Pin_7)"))
 (segment (start 111.14 115.03) (end 111.14 122.21) (width 0.3) (layer "F.Cu") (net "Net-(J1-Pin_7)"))
 (segment (start 156.57 66.68) (end 126.99 66.68) (width 0.3) (layer "F.Cu") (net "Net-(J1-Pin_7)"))
 (segment (start 154.36 124.66) (end 155.95 123.07) (width 0.3) (layer "F.Cu") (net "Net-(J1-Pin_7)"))
 (segment (start 133.53 124.66) (end 154.36 124.66) (width 0.3) (layer "F.Cu") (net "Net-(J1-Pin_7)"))
 (segment (start 133.53 124.32) (end 133.53 124.66) (width 0.3) (layer "F.Cu") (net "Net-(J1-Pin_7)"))
 (segment (start 151.17 118.29) (end 155.95 123.07) (width 0.3) (layer "F.Cu") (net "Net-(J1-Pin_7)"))
 (segment (start 157.3 121.72) (end 157.3 67.41) (width 0.3) (layer "F.Cu") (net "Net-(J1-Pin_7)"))
 (segment (start 126.99 66.68) (end 126.145 65.835) (width 0.3) (layer "F.Cu") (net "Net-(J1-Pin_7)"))
 (segment (start 131.13 121.92) (end 133.53 124.32) (width 0.3) (layer "F.Cu") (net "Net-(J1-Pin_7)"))
 (segment (start 91.13 114.99) (end 91.13 120.58) (width 0.3) (layer "F.Cu") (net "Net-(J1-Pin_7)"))
 (segment (start 151.17 115.09) (end 151.17 118.29) (width 0.3) (layer "F.Cu") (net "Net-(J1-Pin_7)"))
 (segment (start 155.95 123.07) (end 157.3 121.72) (width 0.3) (layer "F.Cu") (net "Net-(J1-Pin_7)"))
 (segment (start 157.3 67.41) (end 156.57 66.68) (width 0.3) (layer "F.Cu") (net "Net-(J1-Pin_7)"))
 (segment (start 133.28 140.47) (end 152.96 140.47) (width 0.3) (layer "F.Cu") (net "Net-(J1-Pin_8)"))
 (segment (start 93.99 140.47) (end 113.52 140.47) (width 0.3) (layer "F.Cu") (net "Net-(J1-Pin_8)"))
 (segment (start 131.14 138.33) (end 133.28 140.47) (width 0.3) (layer "F.Cu") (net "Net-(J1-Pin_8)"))
 (segment (start 158.59 135.05) (end 158.6 135.05) (width 0.3) (layer "F.Cu") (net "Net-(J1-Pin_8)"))
 (segment (start 158.6 66.63) (end 157.67 65.7) (width 0.3) (layer "F.Cu") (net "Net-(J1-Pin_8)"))
 (segment (start 129.41 65.7) (end 128.685 64.975) (width 0.3) (layer "F.Cu") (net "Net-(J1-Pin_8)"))
 (segment (start 152.96 140.47) (end 153.17 140.47) (width 0.3) (layer "F.Cu") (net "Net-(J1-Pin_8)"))
 (segment (start 111.15 138.1) (end 113.52 140.47) (width 0.3) (layer "F.Cu") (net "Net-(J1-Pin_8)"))
 (segment (start 153.17 140.47) (end 158.59 135.05) (width 0.3) (layer "F.Cu") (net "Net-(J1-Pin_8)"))
 (segment (start 91.12 134.51) (end 91.12 137.6) (width 0.3) (layer "F.Cu") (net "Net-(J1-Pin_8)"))
 (segment (start 91.12 137.6) (end 93.99 140.47) (width 0.3) (layer "F.Cu") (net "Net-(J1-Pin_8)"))
 (segment (start 151.17 138.68) (end 152.96 140.47) (width 0.3) (layer "F.Cu") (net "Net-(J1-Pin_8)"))
 (segment (start 111.15 134.58) (end 111.15 138.1) (width 0.3) (layer "F.Cu") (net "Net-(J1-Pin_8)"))
 (segment (start 158.6 135.05) (end 158.6 66.63) (width 0.3) (layer "F.Cu") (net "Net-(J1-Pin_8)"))
 (segment (start 131.14 134.49) (end 131.14 138.33) (width 0.3) (layer "F.Cu") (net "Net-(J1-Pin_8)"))
 (segment (start 113.52 140.47) (end 133.28 140.47) (width 0.3) (layer "F.Cu") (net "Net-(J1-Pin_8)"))
 (segment (start 151.17 134.6) (end 151.17 138.68) (width 0.3) (layer "F.Cu") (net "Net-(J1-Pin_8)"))
 (segment (start 157.67 65.7) (end 129.41 65.7) (width 0.3) (layer "F.Cu") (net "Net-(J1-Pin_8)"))
 (segment (start 88.79 120.36) (end 88.79 109.59) (width 0.3) (layer "F.Cu") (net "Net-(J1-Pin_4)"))
 (segment (start 101.48 113.75) (end 142.71 113.75) (width 0.3) (layer "F.Cu") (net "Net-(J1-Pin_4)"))
 (segment (start 88.79 109.59) (end 89.62 108.76) (width 0.3) (layer "F.Cu") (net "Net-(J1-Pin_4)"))
 (segment (start 142.71 113.75) (end 145.37 111.09) (width 0.3) (layer "F.Cu") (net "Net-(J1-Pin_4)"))
 (segment (start 89.57 88.6) (end 93.87 88.6) (width 0.3) (layer "F.Cu") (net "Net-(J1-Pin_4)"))
 (segment (start 93.152894 81.52) (end 89.12 77.487106) (width 0.3) (layer "F.Cu") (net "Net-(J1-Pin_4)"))
 (segment (start 89.95 74.28) (end 143.05 74.28) (width 0.3) (layer "F.Cu") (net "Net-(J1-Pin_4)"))
 (segment (start 89.12 77.487106) (end 89.12 75.11) (width 0.3) (layer "F.Cu") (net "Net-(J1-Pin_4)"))
 (segment (start 94.53 126.1) (end 88.79 120.36) (width 0.3) (layer "F.Cu") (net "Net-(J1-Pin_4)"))
 (segment (start 91.76 103.1) (end 89.04 100.38) (width 0.3) (layer "F.Cu") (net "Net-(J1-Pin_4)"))
 (segment (start 89.62 108.76) (end 96.49 108.76) (width 0.3) (layer "F.Cu") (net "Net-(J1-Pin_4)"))
 (segment (start 136.42 71.99) (end 134.68 70.25) (width 0.3) (layer "F.Cu") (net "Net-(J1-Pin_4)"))
 (segment (start 99.41 94.14) (end 138.39 94.14) (width 0.3) (layer "F.Cu") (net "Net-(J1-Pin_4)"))
 (segment (start 143.05 74.28) (end 145.34 71.99) (width 0.3) (layer "F.Cu") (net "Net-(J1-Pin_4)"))
 (segment (start 138.39 94.14) (end 142.69 94.14) (width 0.3) (layer "F.Cu") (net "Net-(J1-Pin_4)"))
 (segment (start 143.02 81.52) (end 93.152894 81.52) (width 0.3) (layer "F.Cu") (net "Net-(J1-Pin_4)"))
 (segment (start 138.57 93.96) (end 138.39 94.14) (width 0.3) (layer "F.Cu") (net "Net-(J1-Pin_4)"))
 (segment (start 145.34 83.84) (end 143.02 81.52) (width 0.3) (layer "F.Cu") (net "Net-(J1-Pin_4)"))
 (segment (start 142.69 94.14) (end 145.34 91.49) (width 0.3) (layer "F.Cu") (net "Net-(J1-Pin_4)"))
 (segment (start 145.37 130.6) (end 145.37 128.28) (width 0.3) (layer "F.Cu") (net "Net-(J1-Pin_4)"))
 (segment (start 141.34 103) (end 141.24 103.1) (width 0.3) (layer "F.Cu") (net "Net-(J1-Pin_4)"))
 (segment (start 93.87 88.6) (end 99.41 94.14) (width 0.3) (layer "F.Cu") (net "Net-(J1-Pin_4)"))
 (segment (start 119.96 70.25) (end 134.68 70.25) (width 0.3) (layer "F.Cu") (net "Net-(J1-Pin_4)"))
 (segment (start 145.37 128.28) (end 143.19 126.1) (width 0.3) (layer "F.Cu") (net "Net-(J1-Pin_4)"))
 (segment (start 141.24 103.1) (end 91.76 103.1) (width 0.3) (layer "F.Cu") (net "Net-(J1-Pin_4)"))
 (segment (start 145.37 107.03) (end 141.34 103) (width 0.3) (layer "F.Cu") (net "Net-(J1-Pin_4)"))
 (segment (start 96.49 108.76) (end 101.48 113.75) (width 0.3) (layer "F.Cu") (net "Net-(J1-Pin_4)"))
 (segment (start 145.34 91.49) (end 145.34 83.84) (width 0.3) (layer "F.Cu") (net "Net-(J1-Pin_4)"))
 (segment (start 119.96 66.41) (end 119.96 70.25) (width 0.3) (layer "F.Cu") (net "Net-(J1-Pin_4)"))
 (segment (start 145.37 111.09) (end 145.37 107.03) (width 0.3) (layer "F.Cu") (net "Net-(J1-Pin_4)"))
 (segment (start 89.12 75.11) (end 89.95 74.28) (width 0.3) (layer "F.Cu") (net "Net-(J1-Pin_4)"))
 (segment (start 145.34 71.99) (end 136.42 71.99) (width 0.3) (layer "F.Cu") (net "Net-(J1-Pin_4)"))
 (segment (start 118.525 64.975) (end 119.96 66.41) (width 0.3) (layer "F.Cu") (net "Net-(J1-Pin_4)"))
 (segment (start 89.04 100.38) (end 89.04 89.13) (width 0.3) (layer "F.Cu") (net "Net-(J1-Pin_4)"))
 (segment (start 143.19 126.1) (end 94.53 126.1) (width 0.3) (layer "F.Cu") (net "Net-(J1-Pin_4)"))
 (segment (start 89.04 89.13) (end 89.57 88.6) (width 0.3) (layer "F.Cu") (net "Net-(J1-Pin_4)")))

